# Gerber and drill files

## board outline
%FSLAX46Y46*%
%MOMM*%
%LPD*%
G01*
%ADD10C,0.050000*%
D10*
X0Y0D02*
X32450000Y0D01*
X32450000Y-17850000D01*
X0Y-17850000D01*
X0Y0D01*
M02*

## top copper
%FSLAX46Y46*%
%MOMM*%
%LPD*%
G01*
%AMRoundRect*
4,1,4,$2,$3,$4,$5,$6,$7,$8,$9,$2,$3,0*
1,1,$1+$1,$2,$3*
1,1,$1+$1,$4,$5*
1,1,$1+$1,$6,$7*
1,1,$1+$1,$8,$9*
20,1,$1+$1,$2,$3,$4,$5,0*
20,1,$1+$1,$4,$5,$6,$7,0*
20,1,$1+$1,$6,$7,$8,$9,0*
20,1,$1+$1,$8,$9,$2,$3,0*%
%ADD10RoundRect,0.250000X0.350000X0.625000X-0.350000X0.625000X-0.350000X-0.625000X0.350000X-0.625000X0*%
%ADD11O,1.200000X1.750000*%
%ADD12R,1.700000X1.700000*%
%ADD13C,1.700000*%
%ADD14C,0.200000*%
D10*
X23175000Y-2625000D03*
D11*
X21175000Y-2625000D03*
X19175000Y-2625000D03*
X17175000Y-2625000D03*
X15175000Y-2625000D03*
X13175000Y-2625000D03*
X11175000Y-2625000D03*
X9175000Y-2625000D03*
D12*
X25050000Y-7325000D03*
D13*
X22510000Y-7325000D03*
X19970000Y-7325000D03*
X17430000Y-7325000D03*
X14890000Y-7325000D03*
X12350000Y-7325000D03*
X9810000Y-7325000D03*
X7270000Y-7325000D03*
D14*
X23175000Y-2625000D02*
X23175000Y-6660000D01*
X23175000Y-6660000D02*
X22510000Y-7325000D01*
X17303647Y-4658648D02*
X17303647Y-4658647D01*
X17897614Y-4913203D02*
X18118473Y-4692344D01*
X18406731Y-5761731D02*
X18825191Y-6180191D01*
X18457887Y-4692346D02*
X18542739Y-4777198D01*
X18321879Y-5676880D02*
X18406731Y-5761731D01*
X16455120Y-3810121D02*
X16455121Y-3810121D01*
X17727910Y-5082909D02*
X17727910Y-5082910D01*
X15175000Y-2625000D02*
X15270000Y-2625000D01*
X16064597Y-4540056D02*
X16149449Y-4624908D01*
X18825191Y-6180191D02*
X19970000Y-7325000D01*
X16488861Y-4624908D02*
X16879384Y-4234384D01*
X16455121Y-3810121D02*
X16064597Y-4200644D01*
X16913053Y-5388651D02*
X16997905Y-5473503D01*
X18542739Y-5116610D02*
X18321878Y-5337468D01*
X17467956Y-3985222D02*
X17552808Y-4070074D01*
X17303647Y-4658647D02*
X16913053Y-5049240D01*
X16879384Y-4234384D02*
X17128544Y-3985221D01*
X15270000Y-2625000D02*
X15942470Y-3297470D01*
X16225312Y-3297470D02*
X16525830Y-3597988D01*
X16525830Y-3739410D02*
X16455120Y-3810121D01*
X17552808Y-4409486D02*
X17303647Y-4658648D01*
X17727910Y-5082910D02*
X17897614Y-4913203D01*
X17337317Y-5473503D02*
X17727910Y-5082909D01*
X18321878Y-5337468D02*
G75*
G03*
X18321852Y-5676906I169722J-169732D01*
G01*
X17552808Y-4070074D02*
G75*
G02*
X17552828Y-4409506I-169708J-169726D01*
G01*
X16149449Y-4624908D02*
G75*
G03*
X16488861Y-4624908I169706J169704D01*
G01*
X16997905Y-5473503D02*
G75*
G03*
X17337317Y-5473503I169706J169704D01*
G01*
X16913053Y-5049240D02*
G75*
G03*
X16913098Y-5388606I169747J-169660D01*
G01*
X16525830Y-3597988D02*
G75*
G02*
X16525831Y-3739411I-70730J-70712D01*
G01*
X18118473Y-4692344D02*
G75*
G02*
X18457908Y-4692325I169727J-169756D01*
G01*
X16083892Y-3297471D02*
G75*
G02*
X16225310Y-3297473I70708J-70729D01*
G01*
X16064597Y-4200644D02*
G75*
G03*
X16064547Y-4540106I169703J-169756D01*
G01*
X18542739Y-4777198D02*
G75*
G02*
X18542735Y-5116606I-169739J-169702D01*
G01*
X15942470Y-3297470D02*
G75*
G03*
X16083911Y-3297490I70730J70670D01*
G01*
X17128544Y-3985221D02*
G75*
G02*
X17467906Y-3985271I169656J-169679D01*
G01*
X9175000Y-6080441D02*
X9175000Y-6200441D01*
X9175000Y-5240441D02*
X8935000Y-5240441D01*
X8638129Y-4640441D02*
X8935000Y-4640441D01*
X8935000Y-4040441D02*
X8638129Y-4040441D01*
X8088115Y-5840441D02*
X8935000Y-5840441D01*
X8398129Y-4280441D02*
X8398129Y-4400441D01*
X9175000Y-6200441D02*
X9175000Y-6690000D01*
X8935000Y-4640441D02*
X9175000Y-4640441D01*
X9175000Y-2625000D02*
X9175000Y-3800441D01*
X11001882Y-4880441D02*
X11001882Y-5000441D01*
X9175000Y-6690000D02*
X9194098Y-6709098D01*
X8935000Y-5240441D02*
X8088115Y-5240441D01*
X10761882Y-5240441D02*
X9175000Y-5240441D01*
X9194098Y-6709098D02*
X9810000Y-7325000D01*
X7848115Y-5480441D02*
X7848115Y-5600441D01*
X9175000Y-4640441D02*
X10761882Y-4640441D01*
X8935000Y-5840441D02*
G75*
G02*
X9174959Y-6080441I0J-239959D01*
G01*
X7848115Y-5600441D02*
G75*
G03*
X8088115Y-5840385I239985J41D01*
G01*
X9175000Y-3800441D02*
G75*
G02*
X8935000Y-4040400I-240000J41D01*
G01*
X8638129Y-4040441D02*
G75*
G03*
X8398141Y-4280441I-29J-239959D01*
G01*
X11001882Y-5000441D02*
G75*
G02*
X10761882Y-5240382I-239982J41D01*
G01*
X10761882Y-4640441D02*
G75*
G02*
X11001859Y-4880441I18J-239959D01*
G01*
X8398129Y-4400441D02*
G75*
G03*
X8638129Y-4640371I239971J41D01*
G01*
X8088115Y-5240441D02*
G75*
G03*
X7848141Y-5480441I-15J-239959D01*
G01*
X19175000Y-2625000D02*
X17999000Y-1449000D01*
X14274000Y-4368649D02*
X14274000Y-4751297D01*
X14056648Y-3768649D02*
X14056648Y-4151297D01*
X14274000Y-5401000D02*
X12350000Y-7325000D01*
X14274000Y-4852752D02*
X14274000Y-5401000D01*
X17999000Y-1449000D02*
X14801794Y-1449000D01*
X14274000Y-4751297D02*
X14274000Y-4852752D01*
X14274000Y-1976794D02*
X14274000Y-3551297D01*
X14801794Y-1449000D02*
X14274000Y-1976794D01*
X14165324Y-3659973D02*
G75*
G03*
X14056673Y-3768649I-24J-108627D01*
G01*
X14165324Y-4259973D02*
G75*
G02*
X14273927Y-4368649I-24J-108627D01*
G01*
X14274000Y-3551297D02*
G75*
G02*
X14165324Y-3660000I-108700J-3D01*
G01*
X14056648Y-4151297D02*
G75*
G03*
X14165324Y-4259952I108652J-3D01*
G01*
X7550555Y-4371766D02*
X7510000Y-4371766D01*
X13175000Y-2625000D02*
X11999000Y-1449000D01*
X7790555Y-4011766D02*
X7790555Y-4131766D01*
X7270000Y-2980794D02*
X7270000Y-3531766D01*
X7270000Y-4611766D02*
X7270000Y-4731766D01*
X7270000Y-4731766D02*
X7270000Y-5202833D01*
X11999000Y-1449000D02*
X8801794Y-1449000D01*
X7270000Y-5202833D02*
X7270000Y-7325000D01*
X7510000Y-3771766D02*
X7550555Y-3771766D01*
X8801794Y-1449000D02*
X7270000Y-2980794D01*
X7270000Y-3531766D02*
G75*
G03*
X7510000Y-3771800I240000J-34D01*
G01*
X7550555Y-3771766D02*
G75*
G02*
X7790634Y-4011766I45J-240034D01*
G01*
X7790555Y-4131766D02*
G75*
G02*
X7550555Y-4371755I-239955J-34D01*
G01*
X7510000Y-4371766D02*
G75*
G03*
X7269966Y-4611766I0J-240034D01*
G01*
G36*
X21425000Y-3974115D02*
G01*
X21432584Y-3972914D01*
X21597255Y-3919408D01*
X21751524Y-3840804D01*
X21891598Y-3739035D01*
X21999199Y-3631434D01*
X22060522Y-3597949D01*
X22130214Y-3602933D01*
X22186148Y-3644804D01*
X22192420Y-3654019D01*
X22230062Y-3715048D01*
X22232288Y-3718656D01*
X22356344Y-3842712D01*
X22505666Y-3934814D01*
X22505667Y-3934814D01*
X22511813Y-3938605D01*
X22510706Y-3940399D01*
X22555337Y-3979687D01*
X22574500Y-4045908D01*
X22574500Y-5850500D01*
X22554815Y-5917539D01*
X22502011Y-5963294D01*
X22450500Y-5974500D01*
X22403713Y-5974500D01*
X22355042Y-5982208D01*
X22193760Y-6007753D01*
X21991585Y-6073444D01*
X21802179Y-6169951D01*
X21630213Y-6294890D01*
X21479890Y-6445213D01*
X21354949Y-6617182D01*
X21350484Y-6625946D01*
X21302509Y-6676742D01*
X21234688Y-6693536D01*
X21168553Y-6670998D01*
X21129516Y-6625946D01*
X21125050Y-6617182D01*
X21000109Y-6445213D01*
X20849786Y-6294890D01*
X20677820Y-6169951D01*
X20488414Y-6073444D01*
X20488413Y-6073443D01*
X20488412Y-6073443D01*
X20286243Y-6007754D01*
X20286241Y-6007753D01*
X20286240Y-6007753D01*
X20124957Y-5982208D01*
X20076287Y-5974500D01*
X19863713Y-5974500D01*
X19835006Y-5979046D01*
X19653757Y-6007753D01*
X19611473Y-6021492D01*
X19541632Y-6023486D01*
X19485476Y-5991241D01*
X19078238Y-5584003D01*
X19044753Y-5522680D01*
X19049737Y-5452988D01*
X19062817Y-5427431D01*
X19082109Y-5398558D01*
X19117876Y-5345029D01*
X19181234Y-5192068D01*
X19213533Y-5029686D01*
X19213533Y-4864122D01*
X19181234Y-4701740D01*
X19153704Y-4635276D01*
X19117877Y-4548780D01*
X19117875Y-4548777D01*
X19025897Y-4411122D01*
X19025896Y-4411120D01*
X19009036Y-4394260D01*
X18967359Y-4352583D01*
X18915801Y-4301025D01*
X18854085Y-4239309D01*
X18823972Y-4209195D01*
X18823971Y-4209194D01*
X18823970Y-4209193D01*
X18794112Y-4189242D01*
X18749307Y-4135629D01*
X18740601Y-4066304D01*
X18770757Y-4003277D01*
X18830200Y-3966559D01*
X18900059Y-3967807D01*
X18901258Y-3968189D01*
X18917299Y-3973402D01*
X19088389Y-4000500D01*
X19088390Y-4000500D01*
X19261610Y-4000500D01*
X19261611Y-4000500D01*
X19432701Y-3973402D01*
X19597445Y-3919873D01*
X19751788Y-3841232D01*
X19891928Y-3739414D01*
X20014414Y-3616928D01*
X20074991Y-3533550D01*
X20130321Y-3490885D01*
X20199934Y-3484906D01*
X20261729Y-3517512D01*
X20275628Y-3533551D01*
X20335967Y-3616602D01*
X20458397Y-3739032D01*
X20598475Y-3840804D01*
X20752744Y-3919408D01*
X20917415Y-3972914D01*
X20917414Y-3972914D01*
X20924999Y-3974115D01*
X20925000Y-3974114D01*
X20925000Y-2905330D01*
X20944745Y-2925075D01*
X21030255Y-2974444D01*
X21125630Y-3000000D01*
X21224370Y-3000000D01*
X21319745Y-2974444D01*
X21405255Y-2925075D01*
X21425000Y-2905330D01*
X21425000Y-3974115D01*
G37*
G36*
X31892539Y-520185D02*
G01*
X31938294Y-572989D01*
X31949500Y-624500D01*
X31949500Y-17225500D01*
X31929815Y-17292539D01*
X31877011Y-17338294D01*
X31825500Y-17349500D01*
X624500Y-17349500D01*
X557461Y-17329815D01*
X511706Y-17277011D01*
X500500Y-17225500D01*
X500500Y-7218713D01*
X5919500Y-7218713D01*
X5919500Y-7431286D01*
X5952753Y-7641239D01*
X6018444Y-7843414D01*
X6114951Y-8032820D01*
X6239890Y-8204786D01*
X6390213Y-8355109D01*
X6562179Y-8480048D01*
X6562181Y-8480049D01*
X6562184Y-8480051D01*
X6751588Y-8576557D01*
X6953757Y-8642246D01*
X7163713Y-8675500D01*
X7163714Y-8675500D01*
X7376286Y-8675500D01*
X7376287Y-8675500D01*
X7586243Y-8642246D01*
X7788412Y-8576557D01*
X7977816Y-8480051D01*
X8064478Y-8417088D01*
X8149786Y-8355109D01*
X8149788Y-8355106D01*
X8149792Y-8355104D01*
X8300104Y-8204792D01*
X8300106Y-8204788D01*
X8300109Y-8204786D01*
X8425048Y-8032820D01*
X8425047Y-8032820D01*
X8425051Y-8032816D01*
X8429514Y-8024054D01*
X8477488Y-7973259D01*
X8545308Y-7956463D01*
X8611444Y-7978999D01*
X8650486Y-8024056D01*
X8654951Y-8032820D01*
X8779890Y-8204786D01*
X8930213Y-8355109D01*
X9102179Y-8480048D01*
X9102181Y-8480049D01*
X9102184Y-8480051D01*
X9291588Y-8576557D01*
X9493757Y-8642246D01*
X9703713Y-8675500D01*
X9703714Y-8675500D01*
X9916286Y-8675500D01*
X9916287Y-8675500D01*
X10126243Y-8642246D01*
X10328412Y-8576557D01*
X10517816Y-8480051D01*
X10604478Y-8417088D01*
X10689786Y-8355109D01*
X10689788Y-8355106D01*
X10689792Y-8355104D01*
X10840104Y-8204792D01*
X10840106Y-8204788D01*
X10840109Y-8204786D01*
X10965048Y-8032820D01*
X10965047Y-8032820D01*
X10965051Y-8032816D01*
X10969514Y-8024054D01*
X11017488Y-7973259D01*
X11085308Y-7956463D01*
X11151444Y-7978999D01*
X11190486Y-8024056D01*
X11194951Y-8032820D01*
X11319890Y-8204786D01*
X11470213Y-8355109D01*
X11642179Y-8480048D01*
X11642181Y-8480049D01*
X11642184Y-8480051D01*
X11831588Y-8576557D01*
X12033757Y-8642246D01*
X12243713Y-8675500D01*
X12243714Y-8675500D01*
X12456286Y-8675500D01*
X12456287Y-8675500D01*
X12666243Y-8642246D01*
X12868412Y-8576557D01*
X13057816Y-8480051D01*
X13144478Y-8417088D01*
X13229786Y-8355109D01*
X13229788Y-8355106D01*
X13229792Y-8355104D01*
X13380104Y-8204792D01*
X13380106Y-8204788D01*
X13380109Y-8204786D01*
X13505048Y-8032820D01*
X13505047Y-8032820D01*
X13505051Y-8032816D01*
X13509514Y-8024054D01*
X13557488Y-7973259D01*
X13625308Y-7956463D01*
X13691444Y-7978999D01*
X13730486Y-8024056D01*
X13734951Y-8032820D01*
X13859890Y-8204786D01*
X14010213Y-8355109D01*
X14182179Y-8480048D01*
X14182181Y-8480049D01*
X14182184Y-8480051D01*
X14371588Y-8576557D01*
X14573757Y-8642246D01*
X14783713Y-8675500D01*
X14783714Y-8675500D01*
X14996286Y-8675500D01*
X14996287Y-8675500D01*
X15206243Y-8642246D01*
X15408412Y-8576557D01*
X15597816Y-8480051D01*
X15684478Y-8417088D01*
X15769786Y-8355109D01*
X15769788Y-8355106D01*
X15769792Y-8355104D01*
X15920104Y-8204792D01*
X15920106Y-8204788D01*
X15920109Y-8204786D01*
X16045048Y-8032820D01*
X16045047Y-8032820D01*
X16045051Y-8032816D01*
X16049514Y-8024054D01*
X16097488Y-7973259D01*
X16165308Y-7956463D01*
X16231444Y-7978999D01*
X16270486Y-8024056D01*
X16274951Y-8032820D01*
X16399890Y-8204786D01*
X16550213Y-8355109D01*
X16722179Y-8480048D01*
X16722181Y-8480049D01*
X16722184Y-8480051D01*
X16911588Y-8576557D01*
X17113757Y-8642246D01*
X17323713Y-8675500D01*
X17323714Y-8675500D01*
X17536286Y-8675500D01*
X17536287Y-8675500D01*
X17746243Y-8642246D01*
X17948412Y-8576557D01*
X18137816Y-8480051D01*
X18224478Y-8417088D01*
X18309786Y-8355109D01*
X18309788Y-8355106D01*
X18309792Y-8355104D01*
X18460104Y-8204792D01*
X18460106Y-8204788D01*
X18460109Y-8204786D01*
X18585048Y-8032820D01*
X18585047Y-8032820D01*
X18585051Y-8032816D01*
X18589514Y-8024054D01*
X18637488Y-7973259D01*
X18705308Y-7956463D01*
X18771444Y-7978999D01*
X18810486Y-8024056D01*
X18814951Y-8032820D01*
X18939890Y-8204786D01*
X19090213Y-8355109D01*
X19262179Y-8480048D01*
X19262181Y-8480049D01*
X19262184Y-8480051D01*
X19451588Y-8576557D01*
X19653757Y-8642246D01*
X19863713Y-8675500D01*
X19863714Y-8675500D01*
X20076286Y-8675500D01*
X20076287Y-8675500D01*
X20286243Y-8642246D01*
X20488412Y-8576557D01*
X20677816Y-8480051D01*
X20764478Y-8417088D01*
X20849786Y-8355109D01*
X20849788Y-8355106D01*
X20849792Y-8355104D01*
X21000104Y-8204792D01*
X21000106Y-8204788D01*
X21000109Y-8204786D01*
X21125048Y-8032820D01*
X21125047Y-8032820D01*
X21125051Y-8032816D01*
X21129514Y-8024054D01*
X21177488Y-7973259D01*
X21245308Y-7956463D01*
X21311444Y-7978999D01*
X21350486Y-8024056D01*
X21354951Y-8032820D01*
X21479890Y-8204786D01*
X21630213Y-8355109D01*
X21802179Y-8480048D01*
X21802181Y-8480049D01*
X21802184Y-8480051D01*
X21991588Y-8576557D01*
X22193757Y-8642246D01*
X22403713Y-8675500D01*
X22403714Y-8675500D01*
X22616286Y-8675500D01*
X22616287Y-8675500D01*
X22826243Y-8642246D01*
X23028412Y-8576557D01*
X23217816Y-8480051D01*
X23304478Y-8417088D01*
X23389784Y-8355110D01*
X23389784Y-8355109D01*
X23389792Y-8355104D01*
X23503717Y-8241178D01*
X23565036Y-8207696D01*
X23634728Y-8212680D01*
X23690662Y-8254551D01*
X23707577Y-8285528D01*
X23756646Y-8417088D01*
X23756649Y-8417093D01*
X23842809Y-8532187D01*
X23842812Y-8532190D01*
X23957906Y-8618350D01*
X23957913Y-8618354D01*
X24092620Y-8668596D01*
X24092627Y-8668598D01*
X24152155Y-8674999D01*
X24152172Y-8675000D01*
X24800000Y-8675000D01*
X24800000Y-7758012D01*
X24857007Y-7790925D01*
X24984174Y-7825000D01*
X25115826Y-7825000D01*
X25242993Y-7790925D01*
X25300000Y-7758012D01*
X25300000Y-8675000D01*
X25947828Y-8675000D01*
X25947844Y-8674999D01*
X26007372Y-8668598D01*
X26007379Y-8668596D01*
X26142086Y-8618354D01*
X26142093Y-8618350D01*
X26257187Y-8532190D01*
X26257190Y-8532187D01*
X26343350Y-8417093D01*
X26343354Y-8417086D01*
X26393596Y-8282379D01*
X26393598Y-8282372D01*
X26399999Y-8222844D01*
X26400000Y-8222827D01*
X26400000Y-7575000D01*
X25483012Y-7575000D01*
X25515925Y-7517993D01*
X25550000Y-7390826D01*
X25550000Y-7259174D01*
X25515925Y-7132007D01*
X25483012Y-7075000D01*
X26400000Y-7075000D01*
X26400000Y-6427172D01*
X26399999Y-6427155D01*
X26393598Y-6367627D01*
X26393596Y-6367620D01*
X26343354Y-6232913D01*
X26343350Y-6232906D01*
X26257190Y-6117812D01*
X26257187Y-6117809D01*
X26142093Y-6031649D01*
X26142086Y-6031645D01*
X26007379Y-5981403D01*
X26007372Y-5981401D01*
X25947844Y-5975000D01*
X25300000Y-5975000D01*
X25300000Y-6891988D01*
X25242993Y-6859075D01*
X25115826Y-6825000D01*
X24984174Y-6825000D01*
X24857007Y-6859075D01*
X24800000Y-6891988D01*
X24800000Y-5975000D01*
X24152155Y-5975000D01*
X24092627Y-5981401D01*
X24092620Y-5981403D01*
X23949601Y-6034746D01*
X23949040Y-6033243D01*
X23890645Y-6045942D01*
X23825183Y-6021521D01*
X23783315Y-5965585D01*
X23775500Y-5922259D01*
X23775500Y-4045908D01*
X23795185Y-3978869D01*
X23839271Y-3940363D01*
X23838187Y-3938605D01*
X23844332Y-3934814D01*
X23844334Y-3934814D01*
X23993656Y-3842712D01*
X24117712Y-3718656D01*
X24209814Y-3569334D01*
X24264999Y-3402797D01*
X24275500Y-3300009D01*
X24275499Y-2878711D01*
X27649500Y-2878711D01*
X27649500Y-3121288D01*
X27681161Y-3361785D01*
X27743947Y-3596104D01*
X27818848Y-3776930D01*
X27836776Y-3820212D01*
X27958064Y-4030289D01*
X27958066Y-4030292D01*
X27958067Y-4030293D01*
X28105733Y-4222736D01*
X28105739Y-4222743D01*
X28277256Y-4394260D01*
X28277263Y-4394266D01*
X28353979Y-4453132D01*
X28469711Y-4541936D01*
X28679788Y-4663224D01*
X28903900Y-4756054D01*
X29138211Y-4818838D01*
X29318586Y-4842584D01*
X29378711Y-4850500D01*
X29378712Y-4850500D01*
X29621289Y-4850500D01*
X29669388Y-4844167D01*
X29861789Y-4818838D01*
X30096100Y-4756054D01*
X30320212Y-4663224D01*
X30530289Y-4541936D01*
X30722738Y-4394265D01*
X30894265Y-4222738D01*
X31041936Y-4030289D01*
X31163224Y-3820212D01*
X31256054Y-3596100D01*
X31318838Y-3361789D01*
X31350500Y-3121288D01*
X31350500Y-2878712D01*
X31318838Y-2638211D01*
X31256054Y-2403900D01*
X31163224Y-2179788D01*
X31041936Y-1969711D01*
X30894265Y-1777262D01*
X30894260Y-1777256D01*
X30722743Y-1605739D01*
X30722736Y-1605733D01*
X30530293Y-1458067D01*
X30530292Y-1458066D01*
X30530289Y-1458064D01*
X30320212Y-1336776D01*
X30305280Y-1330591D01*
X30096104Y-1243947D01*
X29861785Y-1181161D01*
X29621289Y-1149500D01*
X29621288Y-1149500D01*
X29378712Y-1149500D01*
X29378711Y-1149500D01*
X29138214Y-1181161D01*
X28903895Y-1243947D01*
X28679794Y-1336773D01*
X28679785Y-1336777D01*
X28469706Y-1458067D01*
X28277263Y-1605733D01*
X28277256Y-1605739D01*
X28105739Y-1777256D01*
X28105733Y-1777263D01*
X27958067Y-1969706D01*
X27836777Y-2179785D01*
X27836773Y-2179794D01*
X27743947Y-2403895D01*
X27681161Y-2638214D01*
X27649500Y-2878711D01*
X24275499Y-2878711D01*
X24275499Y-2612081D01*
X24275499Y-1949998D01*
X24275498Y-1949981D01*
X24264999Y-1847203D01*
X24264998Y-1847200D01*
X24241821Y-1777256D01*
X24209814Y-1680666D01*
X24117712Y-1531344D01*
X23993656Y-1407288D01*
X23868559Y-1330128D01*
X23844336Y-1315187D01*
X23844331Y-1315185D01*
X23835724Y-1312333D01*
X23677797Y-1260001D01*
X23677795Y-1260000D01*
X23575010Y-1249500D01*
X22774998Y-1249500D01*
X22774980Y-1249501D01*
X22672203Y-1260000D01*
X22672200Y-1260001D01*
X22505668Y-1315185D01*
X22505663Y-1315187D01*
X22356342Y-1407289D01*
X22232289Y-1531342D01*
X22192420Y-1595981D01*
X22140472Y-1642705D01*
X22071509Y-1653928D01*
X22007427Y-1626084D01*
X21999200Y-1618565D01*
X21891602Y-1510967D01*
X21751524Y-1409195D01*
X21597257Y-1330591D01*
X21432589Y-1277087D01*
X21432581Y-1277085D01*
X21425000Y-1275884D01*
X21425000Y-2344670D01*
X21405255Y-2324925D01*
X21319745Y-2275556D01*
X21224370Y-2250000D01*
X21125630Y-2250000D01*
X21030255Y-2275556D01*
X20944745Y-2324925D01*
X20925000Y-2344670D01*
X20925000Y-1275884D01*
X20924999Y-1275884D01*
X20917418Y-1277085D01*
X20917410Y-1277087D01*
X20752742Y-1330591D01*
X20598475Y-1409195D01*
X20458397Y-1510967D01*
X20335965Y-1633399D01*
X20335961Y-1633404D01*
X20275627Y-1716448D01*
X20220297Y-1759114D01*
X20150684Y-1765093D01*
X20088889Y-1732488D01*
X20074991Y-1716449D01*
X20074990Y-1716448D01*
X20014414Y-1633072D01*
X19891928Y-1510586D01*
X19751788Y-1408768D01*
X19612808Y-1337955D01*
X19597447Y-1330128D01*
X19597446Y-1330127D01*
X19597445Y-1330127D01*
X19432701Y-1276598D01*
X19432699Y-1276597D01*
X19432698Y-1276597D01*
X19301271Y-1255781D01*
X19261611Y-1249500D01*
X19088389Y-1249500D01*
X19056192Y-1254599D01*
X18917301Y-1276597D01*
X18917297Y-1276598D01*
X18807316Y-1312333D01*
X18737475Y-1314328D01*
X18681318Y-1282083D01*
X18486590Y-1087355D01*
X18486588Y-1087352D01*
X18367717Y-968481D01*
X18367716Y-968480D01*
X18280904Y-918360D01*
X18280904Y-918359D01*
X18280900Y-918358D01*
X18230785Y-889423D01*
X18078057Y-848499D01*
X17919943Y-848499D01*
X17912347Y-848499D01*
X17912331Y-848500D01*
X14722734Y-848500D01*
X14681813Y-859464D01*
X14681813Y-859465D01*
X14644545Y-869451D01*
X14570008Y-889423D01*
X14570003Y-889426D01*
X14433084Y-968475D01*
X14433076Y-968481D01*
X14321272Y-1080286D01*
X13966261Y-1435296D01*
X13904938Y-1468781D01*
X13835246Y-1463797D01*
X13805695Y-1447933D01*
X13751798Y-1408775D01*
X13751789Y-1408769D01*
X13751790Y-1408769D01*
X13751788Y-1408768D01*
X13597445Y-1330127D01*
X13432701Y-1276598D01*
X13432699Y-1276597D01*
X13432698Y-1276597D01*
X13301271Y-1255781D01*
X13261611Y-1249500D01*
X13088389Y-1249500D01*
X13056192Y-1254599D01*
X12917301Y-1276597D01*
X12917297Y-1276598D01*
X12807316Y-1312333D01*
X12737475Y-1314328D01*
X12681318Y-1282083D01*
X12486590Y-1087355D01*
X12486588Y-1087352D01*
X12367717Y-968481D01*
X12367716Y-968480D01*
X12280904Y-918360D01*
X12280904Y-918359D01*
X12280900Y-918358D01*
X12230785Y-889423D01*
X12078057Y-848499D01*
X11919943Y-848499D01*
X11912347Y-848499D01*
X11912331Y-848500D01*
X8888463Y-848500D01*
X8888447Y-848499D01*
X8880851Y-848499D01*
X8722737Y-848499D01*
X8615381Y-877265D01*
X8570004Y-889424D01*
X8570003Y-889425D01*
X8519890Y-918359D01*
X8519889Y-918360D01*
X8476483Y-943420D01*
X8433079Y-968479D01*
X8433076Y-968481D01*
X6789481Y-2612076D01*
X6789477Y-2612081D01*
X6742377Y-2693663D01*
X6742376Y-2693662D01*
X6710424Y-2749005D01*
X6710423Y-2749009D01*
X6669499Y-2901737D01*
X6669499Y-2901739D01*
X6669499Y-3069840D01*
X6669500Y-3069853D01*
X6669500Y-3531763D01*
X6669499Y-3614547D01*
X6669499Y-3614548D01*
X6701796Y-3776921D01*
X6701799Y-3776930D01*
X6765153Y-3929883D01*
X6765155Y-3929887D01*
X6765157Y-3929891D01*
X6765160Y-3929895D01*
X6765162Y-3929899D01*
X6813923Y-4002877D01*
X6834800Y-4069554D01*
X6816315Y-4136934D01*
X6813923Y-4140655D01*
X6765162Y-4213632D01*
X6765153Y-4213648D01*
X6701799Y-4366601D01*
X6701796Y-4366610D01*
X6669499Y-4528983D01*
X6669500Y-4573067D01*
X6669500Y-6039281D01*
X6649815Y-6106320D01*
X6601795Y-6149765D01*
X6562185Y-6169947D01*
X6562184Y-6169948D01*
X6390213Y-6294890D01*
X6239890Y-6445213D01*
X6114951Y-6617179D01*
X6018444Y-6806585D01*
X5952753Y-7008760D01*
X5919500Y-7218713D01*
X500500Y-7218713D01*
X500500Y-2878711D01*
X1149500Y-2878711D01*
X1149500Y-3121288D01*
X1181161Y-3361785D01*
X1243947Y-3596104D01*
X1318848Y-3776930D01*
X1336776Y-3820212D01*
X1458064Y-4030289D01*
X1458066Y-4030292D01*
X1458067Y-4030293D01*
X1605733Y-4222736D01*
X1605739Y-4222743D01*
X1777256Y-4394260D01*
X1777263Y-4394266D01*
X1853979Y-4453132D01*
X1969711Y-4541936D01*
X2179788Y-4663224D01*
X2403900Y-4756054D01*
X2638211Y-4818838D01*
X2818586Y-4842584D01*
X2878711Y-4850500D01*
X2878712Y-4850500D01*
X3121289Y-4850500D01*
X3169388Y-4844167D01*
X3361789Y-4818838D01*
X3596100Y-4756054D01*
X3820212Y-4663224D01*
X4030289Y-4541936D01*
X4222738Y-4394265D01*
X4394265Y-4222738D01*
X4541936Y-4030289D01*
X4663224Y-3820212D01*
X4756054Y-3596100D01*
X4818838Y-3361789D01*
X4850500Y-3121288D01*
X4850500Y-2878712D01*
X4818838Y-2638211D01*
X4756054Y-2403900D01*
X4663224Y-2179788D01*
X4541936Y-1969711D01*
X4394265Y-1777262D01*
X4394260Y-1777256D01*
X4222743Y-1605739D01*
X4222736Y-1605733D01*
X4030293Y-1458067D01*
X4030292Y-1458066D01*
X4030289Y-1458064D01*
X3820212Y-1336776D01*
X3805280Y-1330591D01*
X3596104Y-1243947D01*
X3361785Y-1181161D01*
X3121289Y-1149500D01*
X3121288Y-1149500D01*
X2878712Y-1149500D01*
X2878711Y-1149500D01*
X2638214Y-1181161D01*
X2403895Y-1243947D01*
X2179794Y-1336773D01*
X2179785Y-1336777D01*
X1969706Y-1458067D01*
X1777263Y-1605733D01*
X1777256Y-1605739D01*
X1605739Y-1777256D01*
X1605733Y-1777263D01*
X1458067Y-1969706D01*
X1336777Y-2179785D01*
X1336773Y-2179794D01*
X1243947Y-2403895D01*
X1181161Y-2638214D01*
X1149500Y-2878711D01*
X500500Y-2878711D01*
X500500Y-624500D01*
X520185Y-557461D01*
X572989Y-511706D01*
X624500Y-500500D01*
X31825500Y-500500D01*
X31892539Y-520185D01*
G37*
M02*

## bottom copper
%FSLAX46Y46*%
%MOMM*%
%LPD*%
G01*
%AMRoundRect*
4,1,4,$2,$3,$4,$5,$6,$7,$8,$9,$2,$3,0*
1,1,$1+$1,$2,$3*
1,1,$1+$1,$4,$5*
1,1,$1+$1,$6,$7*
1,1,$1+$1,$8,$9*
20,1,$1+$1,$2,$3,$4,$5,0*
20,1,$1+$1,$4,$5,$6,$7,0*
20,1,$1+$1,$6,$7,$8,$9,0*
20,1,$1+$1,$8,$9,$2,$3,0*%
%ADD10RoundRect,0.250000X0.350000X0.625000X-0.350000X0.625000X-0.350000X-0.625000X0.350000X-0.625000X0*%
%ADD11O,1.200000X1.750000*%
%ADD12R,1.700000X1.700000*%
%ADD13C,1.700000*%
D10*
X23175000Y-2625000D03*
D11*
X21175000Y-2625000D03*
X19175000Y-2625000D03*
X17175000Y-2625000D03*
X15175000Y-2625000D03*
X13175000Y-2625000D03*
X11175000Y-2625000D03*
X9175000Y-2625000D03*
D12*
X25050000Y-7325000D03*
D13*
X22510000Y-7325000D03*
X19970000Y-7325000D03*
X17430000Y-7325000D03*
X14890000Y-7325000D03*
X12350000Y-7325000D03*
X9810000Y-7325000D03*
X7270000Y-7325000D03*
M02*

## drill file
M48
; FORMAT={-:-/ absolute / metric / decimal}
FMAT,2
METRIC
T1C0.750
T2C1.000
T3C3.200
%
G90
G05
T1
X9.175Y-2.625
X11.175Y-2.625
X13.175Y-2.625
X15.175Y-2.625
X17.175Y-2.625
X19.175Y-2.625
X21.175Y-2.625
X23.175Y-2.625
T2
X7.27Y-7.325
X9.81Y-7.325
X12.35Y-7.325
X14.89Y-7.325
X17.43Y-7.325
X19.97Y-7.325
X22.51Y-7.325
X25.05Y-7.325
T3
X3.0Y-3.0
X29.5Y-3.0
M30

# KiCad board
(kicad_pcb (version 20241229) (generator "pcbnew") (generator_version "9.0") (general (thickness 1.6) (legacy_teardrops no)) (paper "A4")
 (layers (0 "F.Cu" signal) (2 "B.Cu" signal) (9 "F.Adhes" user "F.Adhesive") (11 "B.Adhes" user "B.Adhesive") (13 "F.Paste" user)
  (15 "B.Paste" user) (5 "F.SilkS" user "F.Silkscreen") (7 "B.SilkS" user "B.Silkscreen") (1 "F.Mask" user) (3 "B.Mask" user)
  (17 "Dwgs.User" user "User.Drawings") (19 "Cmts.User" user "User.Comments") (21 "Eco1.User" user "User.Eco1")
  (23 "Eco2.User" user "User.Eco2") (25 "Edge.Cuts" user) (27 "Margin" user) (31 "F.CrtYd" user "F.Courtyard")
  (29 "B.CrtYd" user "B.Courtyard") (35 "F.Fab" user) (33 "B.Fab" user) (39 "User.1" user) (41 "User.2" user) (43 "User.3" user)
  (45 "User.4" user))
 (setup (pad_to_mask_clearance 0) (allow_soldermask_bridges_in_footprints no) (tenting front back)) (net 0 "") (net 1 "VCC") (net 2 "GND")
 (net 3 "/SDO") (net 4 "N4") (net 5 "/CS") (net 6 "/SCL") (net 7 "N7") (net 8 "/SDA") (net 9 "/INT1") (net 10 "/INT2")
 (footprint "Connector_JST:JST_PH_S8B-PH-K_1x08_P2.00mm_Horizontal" (layer "F.Cu") (at 23.175 2.625 180)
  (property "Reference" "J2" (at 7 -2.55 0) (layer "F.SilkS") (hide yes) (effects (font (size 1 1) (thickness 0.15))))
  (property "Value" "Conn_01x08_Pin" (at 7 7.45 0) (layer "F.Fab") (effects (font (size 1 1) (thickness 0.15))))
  (pad "1" thru_hole roundrect (at 0 0 180) (size 1.2 1.75) (drill 0.75) (layers "*.Cu" "*.Mask") (remove_unused_layers no)
   (roundrect_rratio 0.208333) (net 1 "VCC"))
  (pad "2" thru_hole oval (at 2 0 180) (size 1.2 1.75) (drill 0.75) (layers "*.Cu" "*.Mask") (remove_unused_layers no) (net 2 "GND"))
  (pad "3" thru_hole oval (at 4 0 180) (size 1.2 1.75) (drill 0.75) (layers "*.Cu" "*.Mask") (remove_unused_layers no) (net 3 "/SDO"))
  (pad "4" thru_hole oval (at 6 0 180) (size 1.2 1.75) (drill 0.75) (layers "*.Cu" "*.Mask") (remove_unused_layers no) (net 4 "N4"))
  (pad "5" thru_hole oval (at 8 0 180) (size 1.2 1.75) (drill 0.75) (layers "*.Cu" "*.Mask") (remove_unused_layers no) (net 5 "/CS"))
  (pad "6" thru_hole oval (at 10 0 180) (size 1.2 1.75) (drill 0.75) (layers "*.Cu" "*.Mask") (remove_unused_layers no) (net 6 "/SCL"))
  (pad "7" thru_hole oval (at 12 0 180) (size 1.2 1.75) (drill 0.75) (layers "*.Cu" "*.Mask") (remove_unused_layers no) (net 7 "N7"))
  (pad "8" thru_hole oval (at 14 0 180) (size 1.2 1.75) (drill 0.75) (layers "*.Cu" "*.Mask") (remove_unused_layers no) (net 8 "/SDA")))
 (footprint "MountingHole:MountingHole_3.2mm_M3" (layer "F.Cu") (at 29.5 3)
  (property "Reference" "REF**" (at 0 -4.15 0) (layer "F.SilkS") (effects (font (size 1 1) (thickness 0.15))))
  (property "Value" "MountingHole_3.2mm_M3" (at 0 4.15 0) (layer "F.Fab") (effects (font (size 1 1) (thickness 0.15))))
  (pad "" np_thru_hole circle (at 0 0) (size 3.2 3.2) (drill 3.2) (layers "*.Cu" "*.Mask")))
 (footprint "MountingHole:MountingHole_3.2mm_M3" (layer "F.Cu") (at 3 3)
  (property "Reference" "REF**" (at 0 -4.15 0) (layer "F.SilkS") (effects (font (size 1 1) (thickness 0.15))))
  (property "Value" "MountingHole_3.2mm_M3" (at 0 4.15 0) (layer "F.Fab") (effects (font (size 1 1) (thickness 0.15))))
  (pad "" np_thru_hole circle (at 0 0) (size 3.2 3.2) (drill 3.2) (layers "*.Cu" "*.Mask")))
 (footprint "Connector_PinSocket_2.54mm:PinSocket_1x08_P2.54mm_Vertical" (layer "F.Cu") (at 25.05 7.325 -90)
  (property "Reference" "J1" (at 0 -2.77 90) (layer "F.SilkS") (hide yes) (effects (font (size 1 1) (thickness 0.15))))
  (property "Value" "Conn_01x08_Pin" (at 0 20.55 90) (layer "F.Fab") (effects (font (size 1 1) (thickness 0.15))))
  (pad "1" thru_hole rect (at 0 0 270) (size 1.7 1.7) (drill 1) (layers "*.Cu" "*.Mask") (remove_unused_layers no) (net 2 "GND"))
  (pad "2" thru_hole circle (at 0 2.54 270) (size 1.7 1.7) (drill 1) (layers "*.Cu" "*.Mask") (remove_unused_layers no) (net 1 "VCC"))
  (pad "3" thru_hole circle (at 0 5.08 270) (size 1.7 1.7) (drill 1) (layers "*.Cu" "*.Mask") (remove_unused_layers no) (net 5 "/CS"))
  (pad "4" thru_hole circle (at 0 7.62 270) (size 1.7 1.7) (drill 1) (layers "*.Cu" "*.Mask") (remove_unused_layers no) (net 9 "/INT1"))
  (pad "5" thru_hole circle (at 0 10.16 270) (size 1.7 1.7) (drill 1) (layers "*.Cu" "*.Mask") (remove_unused_layers no) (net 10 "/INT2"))
  (pad "6" thru_hole circle (at 0 12.7 270) (size 1.7 1.7) (drill 1) (layers "*.Cu" "*.Mask") (remove_unused_layers no) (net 3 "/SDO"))
  (pad "7" thru_hole circle (at 0 15.24 270) (size 1.7 1.7) (drill 1) (layers "*.Cu" "*.Mask") (remove_unused_layers no) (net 8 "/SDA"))
  (pad "8" thru_hole circle (at 0 17.78 270) (size 1.7 1.7) (drill 1) (layers "*.Cu" "*.Mask") (remove_unused_layers no) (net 6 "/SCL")))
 (gr_rect (start 0 0) (end 32.45 17.85) (stroke (width 0.05) (type solid)) (fill no) (layer "Edge.Cuts"))
 (segment (start 23.175 2.625) (end 23.175 6.66) (width 0.2) (layer "F.Cu") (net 1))
 (segment (start 23.175 6.66) (end 22.51 7.325) (width 0.2) (layer "F.Cu") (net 1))
 (segment (start 17.303647 4.658648) (end 17.303647 4.658647) (width 0.2) (layer "F.Cu") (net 5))
 (segment (start 17.897614 4.913203) (end 18.118473 4.692344) (width 0.2) (layer "F.Cu") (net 5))
 (segment (start 18.406731 5.761731) (end 18.825191 6.180191) (width 0.2) (layer "F.Cu") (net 5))
 (segment (start 18.457887 4.692346) (end 18.542739 4.777198) (width 0.2) (layer "F.Cu") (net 5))
 (segment (start 18.321879 5.67688) (end 18.406731 5.761731) (width 0.2) (layer "F.Cu") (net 5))
 (segment (start 16.45512 3.810121) (end 16.455121 3.810121) (width 0.2) (layer "F.Cu") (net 5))
 (segment (start 17.72791 5.082909) (end 17.72791 5.08291) (width 0.2) (layer "F.Cu") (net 5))
 (segment (start 15.175 2.625) (end 15.27 2.625) (width 0.2) (layer "F.Cu") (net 5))
 (segment (start 16.064597 4.540056) (end 16.149449 4.624908) (width 0.2) (layer "F.Cu") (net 5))
 (segment (start 18.825191 6.180191) (end 19.97 7.325) (width 0.2) (layer "F.Cu") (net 5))
 (segment (start 16.488861 4.624908) (end 16.879384 4.234384) (width 0.2) (layer "F.Cu") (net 5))
 (segment (start 16.455121 3.810121) (end 16.064597 4.200644) (width 0.2) (layer "F.Cu") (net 5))
 (segment (start 16.913053 5.388651) (end 16.997905 5.473503) (width 0.2) (layer "F.Cu") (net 5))
 (segment (start 18.542739 5.11661) (end 18.321878 5.337468) (width 0.2) (layer "F.Cu") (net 5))
 (segment (start 17.467956 3.985222) (end 17.552808 4.070074) (width 0.2) (layer "F.Cu") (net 5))
 (segment (start 17.303647 4.658647) (end 16.913053 5.04924) (width 0.2) (layer "F.Cu") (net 5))
 (segment (start 16.879384 4.234384) (end 17.128544 3.985221) (width 0.2) (layer "F.Cu") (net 5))
 (segment (start 15.27 2.625) (end 15.94247 3.29747) (width 0.2) (layer "F.Cu") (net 5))
 (segment (start 16.225312 3.29747) (end 16.52583 3.597988) (width 0.2) (layer "F.Cu") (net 5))
 (segment (start 16.52583 3.73941) (end 16.45512 3.810121) (width 0.2) (layer "F.Cu") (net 5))
 (segment (start 17.552808 4.409486) (end 17.303647 4.658648) (width 0.2) (layer "F.Cu") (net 5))
 (segment (start 17.72791 5.08291) (end 17.897614 4.913203) (width 0.2) (layer "F.Cu") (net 5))
 (segment (start 17.337317 5.473503) (end 17.72791 5.082909) (width 0.2) (layer "F.Cu") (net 5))
 (arc (start 18.321878 5.337468) (mid 18.251585 5.507174) (end 18.321879 5.67688) (width 0.2) (layer "F.Cu") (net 5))
 (arc (start 17.552808 4.070074) (mid 17.623104 4.239781) (end 17.552808 4.409486) (width 0.2) (layer "F.Cu") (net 5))
 (arc (start 16.149449 4.624908) (mid 16.319155 4.695203) (end 16.488861 4.624908) (width 0.2) (layer "F.Cu") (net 5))
 (arc (start 16.997905 5.473503) (mid 17.167611 5.543798) (end 17.337317 5.473503) (width 0.2) (layer "F.Cu") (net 5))
 (arc (start 16.913053 5.04924) (mid 16.842759 5.218945) (end 16.913053 5.388651) (width 0.2) (layer "F.Cu") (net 5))
 (arc (start 16.52583 3.597988) (mid 16.555119 3.668699) (end 16.52583 3.73941) (width 0.2) (layer "F.Cu") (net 5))
 (arc (start 18.118473 4.692344) (mid 18.28818 4.62205) (end 18.457887 4.692346) (width 0.2) (layer "F.Cu") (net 5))
 (arc (start 16.083892 3.297471) (mid 16.154601 3.268181) (end 16.225312 3.29747) (width 0.2) (layer "F.Cu") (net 5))
 (arc (start 16.064597 4.200644) (mid 15.994302 4.37035) (end 16.064597 4.540056) (width 0.2) (layer "F.Cu") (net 5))
 (arc (start 18.542739 4.777198) (mid 18.613033 4.946903) (end 18.542739 5.11661) (width 0.2) (layer "F.Cu") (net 5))
 (arc (start 15.94247 3.29747) (mid 16.013181 3.326759) (end 16.083892 3.297471) (width 0.2) (layer "F.Cu") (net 5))
 (arc (start 17.128544 3.985221) (mid 17.29825 3.914928) (end 17.467956 3.985222) (width 0.2) (layer "F.Cu") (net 5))
 (segment (start 9.175 6.080441) (end 9.175 6.200441) (width 0.2) (layer "F.Cu") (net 8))
 (segment (start 9.175 5.240441) (end 8.935 5.240441) (width 0.2) (layer "F.Cu") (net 8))
 (segment (start 8.638129 4.640441) (end 8.935 4.640441) (width 0.2) (layer "F.Cu") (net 8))
 (segment (start 8.935 4.040441) (end 8.638129 4.040441) (width 0.2) (layer "F.Cu") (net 8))
 (segment (start 8.088115 5.840441) (end 8.935 5.840441) (width 0.2) (layer "F.Cu") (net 8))
 (segment (start 8.398129 4.280441) (end 8.398129 4.400441) (width 0.2) (layer "F.Cu") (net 8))
 (segment (start 9.175 6.200441) (end 9.175 6.69) (width 0.2) (layer "F.Cu") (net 8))
 (segment (start 8.935 4.640441) (end 9.175 4.640441) (width 0.2) (layer "F.Cu") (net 8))
 (segment (start 9.175 2.625) (end 9.175 3.800441) (width 0.2) (layer "F.Cu") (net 8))
 (segment (start 11.001882 4.880441) (end 11.001882 5.000441) (width 0.2) (layer "F.Cu") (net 8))
 (segment (start 9.175 6.69) (end 9.194098 6.709098) (width 0.2) (layer "F.Cu") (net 8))
 (segment (start 8.935 5.240441) (end 8.088115 5.240441) (width 0.2) (layer "F.Cu") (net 8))
 (segment (start 10.761882 5.240441) (end 9.175 5.240441) (width 0.2) (layer "F.Cu") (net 8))
 (segment (start 9.194098 6.709098) (end 9.81 7.325) (width 0.2) (layer "F.Cu") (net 8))
 (segment (start 7.848115 5.480441) (end 7.848115 5.600441) (width 0.2) (layer "F.Cu") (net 8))
 (segment (start 9.175 4.640441) (end 10.761882 4.640441) (width 0.2) (layer "F.Cu") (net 8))
 (arc (start 8.935 5.840441) (mid 9.104706 5.910735) (end 9.175 6.080441) (width 0.2) (layer "F.Cu") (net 8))
 (arc (start 7.848115 5.600441) (mid 7.918409 5.770147) (end 8.088115 5.840441) (width 0.2) (layer "F.Cu") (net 8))
 (arc (start 9.175 3.800441) (mid 9.104706 3.970147) (end 8.935 4.040441) (width 0.2) (layer "F.Cu") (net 8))
 (arc (start 8.638129 4.040441) (mid 8.468423 4.110735) (end 8.398129 4.280441) (width 0.2) (layer "F.Cu") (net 8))
 (arc (start 11.001882 5.000441) (mid 10.931588 5.170147) (end 10.761882 5.240441) (width 0.2) (layer "F.Cu") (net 8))
 (arc (start 10.761882 4.640441) (mid 10.931588 4.710735) (end 11.001882 4.880441) (width 0.2) (layer "F.Cu") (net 8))
 (arc (start 8.398129 4.400441) (mid 8.468423 4.570147) (end 8.638129 4.640441) (width 0.2) (layer "F.Cu") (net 8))
 (arc (start 8.088115 5.240441) (mid 7.918409 5.310735) (end 7.848115 5.480441) (width 0.2) (layer "F.Cu") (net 8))
 (segment (start 19.175 2.625) (end 17.999 1.449) (width 0.2) (layer "F.Cu") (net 3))
 (segment (start 14.274 4.368649) (end 14.274 4.751297) (width 0.2) (layer "F.Cu") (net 3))
 (segment (start 14.056648 3.768649) (end 14.056648 4.151297) (width 0.2) (layer "F.Cu") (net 3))
 (segment (start 14.274 5.401) (end 12.35 7.325) (width 0.2) (layer "F.Cu") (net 3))
 (segment (start 14.274 4.852752) (end 14.274 5.401) (width 0.2) (layer "F.Cu") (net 3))
 (segment (start 17.999 1.449) (end 14.801794 1.449) (width 0.2) (layer "F.Cu") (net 3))
 (segment (start 14.274 4.751297) (end 14.274 4.852752) (width 0.2) (layer "F.Cu") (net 3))
 (segment (start 14.274 1.976794) (end 14.274 3.551297) (width 0.2) (layer "F.Cu") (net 3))
 (segment (start 14.801794 1.449) (end 14.274 1.976794) (width 0.2) (layer "F.Cu") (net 3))
 (arc (start 14.165324 3.659973) (mid 14.088478 3.691803) (end 14.056648 3.768649) (width 0.2) (layer "F.Cu") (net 3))
 (arc (start 14.165324 4.259973) (mid 14.24217 4.291803) (end 14.274 4.368649) (width 0.2) (layer "F.Cu") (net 3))
 (arc (start 14.274 3.551297) (mid 14.24217 3.628143) (end 14.165324 3.659973) (width 0.2) (layer "F.Cu") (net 3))
 (arc (start 14.056648 4.151297) (mid 14.088478 4.228143) (end 14.165324 4.259973) (width 0.2) (layer "F.Cu") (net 3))
 (segment (start 7.550555 4.371766) (end 7.51 4.371766) (width 0.2) (layer "F.Cu") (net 6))
 (segment (start 13.175 2.625) (end 11.999 1.449) (width 0.2) (layer "F.Cu") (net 6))
 (segment (start 7.790555 4.011766) (end 7.790555 4.131766) (width 0.2) (layer "F.Cu") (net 6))
 (segment (start 7.27 2.980794) (end 7.27 3.531766) (width 0.2) (layer "F.Cu") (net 6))
 (segment (start 7.27 4.611766) (end 7.27 4.731766) (width 0.2) (layer "F.Cu") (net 6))
 (segment (start 7.27 4.731766) (end 7.27 5.202833) (width 0.2) (layer "F.Cu") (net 6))
 (segment (start 11.999 1.449) (end 8.801794 1.449) (width 0.2) (layer "F.Cu") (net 6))
 (segment (start 7.27 5.202833) (end 7.27 7.325) (width 0.2) (layer "F.Cu") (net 6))
 (segment (start 7.51 3.771766) (end 7.550555 3.771766) (width 0.2) (layer "F.Cu") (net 6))
 (segment (start 8.801794 1.449) (end 7.27 2.980794) (width 0.2) (layer "F.Cu") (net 6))
 (arc (start 7.27 3.531766) (mid 7.340294 3.701472) (end 7.51 3.771766) (width 0.2) (layer "F.Cu") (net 6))
 (arc (start 7.550555 3.771766) (mid 7.720261 3.84206) (end 7.790555 4.011766) (width 0.2) (layer "F.Cu") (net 6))
 (arc (start 7.790555 4.131766) (mid 7.720261 4.301472) (end 7.550555 4.371766) (width 0.2) (layer "F.Cu") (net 6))
 (arc (start 7.51 4.371766) (mid 7.340294 4.44206) (end 7.27 4.611766) (width 0.2) (layer "F.Cu") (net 6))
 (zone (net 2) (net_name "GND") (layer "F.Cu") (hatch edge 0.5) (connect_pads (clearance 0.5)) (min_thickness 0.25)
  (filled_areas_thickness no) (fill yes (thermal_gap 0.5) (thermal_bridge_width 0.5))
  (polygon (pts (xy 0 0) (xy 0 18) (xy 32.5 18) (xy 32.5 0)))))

